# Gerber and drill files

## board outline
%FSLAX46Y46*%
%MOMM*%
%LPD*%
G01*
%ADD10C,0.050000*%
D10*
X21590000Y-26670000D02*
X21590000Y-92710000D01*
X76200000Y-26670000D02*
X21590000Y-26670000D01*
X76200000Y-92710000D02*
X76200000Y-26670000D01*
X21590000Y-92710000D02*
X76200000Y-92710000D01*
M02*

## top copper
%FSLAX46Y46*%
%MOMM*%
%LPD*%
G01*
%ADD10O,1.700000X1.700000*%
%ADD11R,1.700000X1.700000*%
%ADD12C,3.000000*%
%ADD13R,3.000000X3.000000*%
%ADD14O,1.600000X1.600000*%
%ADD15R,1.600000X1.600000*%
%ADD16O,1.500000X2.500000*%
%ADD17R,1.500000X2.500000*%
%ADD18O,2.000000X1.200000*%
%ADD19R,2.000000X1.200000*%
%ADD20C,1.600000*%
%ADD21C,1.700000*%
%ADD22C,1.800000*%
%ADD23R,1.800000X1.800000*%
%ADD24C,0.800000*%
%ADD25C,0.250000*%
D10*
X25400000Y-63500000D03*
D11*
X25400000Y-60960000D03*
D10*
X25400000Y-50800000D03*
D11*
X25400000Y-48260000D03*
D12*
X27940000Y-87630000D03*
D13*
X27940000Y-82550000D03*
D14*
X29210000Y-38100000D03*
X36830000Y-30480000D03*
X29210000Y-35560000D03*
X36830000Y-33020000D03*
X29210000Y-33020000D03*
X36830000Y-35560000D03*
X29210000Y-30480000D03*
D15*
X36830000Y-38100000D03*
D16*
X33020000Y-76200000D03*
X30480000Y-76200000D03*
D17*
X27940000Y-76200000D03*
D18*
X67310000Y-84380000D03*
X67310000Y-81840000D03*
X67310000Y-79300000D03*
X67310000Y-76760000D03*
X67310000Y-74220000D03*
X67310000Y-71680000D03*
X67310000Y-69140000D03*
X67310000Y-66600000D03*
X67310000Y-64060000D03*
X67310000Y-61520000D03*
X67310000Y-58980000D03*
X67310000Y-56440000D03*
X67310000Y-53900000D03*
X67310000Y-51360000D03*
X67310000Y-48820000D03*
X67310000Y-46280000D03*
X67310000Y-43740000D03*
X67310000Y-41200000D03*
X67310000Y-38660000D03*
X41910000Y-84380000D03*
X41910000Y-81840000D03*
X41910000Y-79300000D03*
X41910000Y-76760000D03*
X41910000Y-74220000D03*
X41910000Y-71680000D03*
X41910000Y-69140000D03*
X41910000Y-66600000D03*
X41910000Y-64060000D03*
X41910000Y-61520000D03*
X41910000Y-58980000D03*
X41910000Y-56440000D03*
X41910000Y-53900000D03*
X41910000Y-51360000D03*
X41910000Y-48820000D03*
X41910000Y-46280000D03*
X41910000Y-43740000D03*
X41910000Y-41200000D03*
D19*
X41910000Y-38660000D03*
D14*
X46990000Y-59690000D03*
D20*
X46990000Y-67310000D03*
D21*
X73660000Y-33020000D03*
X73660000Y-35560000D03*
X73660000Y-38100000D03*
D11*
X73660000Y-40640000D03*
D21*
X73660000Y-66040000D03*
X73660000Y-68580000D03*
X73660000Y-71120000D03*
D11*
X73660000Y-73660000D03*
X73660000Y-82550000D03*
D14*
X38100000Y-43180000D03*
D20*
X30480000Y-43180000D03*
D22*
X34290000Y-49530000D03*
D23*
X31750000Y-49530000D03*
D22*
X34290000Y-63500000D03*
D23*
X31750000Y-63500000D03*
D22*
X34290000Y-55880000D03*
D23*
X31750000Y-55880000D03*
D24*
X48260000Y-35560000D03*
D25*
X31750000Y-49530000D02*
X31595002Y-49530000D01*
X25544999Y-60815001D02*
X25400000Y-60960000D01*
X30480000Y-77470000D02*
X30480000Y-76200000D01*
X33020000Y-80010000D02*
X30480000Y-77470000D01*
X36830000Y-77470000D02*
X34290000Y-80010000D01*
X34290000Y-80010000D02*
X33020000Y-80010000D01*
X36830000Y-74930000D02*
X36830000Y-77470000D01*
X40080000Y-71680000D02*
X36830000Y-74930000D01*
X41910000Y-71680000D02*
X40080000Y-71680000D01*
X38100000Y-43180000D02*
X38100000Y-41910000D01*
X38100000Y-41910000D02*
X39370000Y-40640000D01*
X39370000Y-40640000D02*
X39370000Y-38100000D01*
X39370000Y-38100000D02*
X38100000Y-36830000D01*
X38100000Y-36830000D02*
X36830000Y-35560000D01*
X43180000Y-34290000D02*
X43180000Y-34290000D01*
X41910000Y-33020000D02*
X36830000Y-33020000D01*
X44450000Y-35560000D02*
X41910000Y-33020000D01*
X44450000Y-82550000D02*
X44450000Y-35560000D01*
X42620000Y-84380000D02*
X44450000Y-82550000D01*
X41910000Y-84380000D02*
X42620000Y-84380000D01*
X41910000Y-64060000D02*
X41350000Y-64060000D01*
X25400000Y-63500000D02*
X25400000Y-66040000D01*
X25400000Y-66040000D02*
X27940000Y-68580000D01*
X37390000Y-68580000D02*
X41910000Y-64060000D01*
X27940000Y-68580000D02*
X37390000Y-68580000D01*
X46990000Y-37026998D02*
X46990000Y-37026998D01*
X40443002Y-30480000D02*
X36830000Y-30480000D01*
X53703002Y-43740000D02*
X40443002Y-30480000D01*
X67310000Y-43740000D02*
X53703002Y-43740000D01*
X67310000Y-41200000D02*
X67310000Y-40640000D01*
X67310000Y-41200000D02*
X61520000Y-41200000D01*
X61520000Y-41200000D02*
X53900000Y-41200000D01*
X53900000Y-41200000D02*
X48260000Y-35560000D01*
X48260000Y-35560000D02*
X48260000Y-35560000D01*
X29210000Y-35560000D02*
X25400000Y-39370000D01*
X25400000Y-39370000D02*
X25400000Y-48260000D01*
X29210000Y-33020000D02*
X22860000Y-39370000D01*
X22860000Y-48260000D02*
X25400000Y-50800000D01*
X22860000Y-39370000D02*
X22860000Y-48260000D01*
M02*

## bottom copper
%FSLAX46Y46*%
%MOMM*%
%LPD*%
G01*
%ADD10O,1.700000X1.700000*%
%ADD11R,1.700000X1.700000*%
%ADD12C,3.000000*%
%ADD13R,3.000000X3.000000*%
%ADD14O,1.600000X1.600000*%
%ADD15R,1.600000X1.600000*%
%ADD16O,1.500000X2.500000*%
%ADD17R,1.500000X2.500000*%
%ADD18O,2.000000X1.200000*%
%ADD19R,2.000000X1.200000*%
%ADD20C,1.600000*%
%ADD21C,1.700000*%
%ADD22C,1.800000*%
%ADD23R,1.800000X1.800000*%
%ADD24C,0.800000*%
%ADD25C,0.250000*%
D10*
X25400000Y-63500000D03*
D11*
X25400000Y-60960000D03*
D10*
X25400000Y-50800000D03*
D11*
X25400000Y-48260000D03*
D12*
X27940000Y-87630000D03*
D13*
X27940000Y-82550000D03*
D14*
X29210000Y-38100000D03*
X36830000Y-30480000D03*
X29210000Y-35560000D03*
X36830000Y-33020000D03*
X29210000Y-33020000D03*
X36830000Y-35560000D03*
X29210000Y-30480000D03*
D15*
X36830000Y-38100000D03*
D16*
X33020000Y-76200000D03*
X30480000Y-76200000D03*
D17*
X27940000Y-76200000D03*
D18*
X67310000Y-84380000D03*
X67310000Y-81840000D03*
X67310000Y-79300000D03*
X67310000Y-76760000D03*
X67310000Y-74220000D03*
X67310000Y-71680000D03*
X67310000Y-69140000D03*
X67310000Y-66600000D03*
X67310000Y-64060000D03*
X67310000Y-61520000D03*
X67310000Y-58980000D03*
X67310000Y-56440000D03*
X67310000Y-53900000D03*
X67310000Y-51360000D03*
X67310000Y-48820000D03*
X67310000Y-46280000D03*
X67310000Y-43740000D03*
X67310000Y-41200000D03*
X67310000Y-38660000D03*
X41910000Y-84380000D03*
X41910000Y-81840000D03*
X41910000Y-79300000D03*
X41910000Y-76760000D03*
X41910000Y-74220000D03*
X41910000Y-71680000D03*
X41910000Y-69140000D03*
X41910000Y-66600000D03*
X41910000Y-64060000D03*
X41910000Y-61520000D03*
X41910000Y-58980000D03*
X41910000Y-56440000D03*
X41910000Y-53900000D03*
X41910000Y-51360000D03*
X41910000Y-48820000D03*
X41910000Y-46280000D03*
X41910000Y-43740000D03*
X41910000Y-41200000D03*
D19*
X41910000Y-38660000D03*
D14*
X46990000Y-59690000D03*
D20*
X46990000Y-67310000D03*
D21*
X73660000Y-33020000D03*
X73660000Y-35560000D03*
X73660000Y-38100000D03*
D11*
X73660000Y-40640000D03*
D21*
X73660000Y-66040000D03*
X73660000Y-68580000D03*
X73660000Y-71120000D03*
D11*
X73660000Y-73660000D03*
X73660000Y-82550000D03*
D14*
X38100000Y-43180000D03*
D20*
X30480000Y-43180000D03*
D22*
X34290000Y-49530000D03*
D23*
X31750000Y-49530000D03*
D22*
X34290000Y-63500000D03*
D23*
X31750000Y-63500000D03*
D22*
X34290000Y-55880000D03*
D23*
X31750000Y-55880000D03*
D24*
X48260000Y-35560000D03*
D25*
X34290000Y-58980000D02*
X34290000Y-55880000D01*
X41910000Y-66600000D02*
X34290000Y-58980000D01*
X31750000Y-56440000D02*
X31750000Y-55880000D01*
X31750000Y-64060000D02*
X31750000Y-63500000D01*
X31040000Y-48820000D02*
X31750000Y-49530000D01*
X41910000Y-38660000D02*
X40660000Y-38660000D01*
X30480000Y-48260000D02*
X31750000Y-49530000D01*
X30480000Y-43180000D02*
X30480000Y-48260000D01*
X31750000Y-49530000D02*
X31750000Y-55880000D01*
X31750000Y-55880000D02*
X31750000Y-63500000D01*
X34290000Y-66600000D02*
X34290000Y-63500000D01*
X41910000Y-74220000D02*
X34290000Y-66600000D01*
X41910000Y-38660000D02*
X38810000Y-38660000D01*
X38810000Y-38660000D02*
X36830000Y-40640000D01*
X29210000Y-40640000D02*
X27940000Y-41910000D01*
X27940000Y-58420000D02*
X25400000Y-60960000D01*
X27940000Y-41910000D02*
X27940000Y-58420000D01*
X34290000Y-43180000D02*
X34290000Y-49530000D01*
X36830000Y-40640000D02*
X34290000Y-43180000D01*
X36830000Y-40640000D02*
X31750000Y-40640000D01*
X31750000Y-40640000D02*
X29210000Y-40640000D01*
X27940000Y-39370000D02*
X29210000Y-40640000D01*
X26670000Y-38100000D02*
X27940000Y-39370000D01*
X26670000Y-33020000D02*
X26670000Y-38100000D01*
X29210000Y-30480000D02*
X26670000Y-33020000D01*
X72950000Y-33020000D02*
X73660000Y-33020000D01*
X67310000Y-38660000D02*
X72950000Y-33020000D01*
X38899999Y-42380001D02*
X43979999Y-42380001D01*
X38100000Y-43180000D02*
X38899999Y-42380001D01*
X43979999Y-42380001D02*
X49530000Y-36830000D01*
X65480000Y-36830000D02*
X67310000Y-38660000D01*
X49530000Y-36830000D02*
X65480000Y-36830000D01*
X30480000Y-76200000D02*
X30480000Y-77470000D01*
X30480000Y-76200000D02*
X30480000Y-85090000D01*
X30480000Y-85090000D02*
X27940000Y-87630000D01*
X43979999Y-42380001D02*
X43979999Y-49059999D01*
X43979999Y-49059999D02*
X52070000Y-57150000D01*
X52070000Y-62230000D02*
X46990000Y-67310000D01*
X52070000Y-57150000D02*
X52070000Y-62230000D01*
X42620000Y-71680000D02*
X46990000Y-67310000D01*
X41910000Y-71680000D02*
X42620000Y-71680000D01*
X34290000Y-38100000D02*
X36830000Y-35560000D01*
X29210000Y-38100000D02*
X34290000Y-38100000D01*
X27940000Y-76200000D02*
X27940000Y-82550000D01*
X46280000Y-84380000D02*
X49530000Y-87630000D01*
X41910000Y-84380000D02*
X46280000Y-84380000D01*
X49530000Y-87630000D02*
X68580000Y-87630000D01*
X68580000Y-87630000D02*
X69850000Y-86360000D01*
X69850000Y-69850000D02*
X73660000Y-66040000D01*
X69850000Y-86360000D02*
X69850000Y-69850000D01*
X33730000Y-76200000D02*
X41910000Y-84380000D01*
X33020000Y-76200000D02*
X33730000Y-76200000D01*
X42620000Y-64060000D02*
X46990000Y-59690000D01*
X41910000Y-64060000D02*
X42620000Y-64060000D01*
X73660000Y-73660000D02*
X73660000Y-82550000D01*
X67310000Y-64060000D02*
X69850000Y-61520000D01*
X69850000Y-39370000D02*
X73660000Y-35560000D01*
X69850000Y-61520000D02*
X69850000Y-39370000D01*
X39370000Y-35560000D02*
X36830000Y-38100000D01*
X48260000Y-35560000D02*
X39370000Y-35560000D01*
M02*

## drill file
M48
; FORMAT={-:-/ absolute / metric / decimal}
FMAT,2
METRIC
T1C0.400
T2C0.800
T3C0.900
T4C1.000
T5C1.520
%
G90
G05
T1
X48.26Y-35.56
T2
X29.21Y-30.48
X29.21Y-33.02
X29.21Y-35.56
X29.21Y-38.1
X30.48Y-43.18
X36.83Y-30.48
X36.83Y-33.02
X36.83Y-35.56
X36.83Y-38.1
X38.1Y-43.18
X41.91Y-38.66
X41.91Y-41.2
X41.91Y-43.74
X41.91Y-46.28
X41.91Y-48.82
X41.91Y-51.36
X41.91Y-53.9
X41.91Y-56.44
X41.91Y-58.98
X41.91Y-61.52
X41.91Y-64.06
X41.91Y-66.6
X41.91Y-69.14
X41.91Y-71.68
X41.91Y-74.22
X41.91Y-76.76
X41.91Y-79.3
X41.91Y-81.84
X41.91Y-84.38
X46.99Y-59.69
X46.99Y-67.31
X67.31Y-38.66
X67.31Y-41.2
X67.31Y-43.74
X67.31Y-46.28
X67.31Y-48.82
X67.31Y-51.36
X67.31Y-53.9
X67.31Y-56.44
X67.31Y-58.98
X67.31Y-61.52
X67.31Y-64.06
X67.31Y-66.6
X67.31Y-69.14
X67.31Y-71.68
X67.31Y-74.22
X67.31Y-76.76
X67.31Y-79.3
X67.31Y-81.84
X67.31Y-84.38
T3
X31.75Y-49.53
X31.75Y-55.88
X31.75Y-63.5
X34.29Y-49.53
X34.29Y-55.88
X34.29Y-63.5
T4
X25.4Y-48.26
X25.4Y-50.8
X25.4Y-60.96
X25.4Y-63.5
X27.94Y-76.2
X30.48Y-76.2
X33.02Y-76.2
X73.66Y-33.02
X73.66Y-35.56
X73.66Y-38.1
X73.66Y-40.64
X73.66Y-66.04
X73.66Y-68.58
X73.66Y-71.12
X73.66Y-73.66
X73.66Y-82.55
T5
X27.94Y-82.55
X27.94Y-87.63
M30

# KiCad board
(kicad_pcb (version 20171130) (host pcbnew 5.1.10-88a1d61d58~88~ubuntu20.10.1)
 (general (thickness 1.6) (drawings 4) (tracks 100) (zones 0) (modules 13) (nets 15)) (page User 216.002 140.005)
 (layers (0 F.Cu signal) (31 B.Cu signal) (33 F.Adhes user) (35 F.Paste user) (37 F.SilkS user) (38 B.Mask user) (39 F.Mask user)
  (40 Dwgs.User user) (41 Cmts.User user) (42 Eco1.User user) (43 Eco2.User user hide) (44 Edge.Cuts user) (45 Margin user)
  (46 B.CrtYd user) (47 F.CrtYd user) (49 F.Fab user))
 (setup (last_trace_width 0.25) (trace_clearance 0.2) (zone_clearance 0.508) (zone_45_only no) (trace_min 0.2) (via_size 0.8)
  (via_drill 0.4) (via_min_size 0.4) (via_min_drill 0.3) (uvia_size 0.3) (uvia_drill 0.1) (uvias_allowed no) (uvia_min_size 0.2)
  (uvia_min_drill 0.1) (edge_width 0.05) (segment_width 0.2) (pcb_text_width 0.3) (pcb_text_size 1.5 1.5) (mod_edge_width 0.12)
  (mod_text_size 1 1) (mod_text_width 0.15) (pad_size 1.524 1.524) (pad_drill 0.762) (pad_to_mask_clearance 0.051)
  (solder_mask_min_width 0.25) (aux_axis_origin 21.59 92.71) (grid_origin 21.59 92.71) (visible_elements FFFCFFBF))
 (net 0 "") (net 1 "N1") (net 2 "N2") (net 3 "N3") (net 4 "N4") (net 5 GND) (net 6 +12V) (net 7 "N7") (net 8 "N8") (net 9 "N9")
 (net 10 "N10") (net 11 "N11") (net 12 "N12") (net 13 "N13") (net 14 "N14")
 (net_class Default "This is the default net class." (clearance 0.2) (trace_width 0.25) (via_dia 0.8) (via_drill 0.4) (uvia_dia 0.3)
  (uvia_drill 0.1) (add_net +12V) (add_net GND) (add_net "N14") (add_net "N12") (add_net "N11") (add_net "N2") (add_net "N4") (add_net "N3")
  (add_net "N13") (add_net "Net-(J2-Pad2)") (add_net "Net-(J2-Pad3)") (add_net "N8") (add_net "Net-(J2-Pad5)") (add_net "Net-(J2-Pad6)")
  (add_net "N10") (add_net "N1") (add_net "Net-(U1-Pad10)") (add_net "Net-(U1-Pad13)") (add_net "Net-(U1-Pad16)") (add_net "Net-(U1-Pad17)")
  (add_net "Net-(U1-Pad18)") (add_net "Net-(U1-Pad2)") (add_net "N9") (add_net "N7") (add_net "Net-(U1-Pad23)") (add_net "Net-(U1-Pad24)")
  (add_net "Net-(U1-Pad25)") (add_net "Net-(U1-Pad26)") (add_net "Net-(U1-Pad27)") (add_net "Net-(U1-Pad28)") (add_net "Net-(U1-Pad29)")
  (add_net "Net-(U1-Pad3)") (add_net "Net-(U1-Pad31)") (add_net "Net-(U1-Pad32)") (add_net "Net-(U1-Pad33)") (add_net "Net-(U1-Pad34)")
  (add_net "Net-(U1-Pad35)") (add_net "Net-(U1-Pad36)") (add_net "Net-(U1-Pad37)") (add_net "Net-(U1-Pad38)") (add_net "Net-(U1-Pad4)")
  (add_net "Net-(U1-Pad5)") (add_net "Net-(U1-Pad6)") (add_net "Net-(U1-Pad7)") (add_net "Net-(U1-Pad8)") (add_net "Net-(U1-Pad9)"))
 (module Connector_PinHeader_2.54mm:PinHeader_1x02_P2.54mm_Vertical (layer F.Cu) (at 25.4 60.96)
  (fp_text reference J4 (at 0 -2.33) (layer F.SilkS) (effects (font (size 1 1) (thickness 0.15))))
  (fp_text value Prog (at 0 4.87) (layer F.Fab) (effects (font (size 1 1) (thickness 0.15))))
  (pad 2 thru_hole oval (at 0 2.54) (size 1.7 1.7) (drill 1) (layers *.Cu *.Mask) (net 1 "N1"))
  (pad 1 thru_hole rect (at 0 0) (size 1.7 1.7) (drill 1) (layers *.Cu *.Mask) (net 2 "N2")))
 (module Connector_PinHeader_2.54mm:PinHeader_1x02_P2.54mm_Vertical (layer F.Cu) (at 25.4 48.26)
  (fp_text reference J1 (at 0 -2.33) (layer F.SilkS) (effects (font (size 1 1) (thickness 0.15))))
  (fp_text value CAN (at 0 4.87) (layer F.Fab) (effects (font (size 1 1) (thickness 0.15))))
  (pad 2 thru_hole oval (at 0 2.54) (size 1.7 1.7) (drill 1) (layers *.Cu *.Mask) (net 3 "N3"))
  (pad 1 thru_hole rect (at 0 0) (size 1.7 1.7) (drill 1) (layers *.Cu *.Mask) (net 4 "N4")))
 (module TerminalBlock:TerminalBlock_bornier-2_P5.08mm (layer F.Cu) (at 27.94 82.55 270)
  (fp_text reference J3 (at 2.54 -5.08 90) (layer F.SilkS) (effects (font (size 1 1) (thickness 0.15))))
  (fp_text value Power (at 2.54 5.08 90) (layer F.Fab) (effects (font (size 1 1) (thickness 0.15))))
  (pad 2 thru_hole circle (at 5.08 0 270) (size 3 3) (drill 1.52) (layers *.Cu *.Mask) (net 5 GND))
  (pad 1 thru_hole rect (at 0 0 270) (size 3 3) (drill 1.52) (layers *.Cu *.Mask) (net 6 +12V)))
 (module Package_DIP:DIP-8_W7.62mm (layer F.Cu) (at 36.83 38.1 180)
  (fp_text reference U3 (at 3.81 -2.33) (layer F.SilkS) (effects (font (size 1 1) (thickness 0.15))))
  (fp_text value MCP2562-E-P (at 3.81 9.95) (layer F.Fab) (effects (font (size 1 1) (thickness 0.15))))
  (pad 8 thru_hole oval (at 7.62 0 180) (size 1.6 1.6) (drill 0.8) (layers *.Cu *.Mask) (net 5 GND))
  (pad 4 thru_hole oval (at 0 7.62 180) (size 1.6 1.6) (drill 0.8) (layers *.Cu *.Mask) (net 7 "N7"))
  (pad 7 thru_hole oval (at 7.62 2.54 180) (size 1.6 1.6) (drill 0.8) (layers *.Cu *.Mask) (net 4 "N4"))
  (pad 3 thru_hole oval (at 0 5.08 180) (size 1.6 1.6) (drill 0.8) (layers *.Cu *.Mask) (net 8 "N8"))
  (pad 6 thru_hole oval (at 7.62 5.08 180) (size 1.6 1.6) (drill 0.8) (layers *.Cu *.Mask) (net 3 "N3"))
  (pad 2 thru_hole oval (at 0 2.54 180) (size 1.6 1.6) (drill 0.8) (layers *.Cu *.Mask) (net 5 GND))
  (pad 5 thru_hole oval (at 7.62 7.62 180) (size 1.6 1.6) (drill 0.8) (layers *.Cu *.Mask) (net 2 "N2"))
  (pad 1 thru_hole rect (at 0 0 180) (size 1.6 1.6) (drill 0.8) (layers *.Cu *.Mask) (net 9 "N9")))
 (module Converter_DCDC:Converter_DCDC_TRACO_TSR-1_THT (layer F.Cu) (at 27.94 76.2)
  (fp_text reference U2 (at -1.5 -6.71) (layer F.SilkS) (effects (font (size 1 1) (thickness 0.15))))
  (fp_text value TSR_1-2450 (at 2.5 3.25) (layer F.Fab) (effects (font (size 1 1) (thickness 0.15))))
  (pad 3 thru_hole oval (at 5.08 0) (size 1.5 2.5) (drill 1) (layers *.Cu *.Mask) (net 8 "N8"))
  (pad 2 thru_hole oval (at 2.54 0) (size 1.5 2.5) (drill 1) (layers *.Cu *.Mask) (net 5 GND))
  (pad 1 thru_hole rect (at 0 0) (size 1.5 2.5) (drill 1) (layers *.Cu *.Mask) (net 6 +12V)))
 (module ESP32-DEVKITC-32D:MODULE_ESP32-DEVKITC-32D (layer F.Cu) (at 54.61 58.42)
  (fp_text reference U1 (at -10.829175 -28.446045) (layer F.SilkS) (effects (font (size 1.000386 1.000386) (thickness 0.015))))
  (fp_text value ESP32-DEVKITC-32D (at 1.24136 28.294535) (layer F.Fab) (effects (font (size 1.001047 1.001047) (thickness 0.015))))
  (pad 38 thru_hole oval (at 12.7 25.96) (size 2 1.2) (drill 0.8) (layers *.Cu *.Mask))
  (pad 37 thru_hole oval (at 12.7 23.42) (size 2 1.2) (drill 0.8) (layers *.Cu *.Mask))
  (pad 36 thru_hole oval (at 12.7 20.88) (size 2 1.2) (drill 0.8) (layers *.Cu *.Mask))
  (pad 35 thru_hole oval (at 12.7 18.34) (size 2 1.2) (drill 0.8) (layers *.Cu *.Mask))
  (pad 34 thru_hole oval (at 12.7 15.8) (size 2 1.2) (drill 0.8) (layers *.Cu *.Mask))
  (pad 33 thru_hole oval (at 12.7 13.26) (size 2 1.2) (drill 0.8) (layers *.Cu *.Mask))
  (pad 32 thru_hole oval (at 12.7 10.72) (size 2 1.2) (drill 0.8) (layers *.Cu *.Mask))
  (pad 31 thru_hole oval (at 12.7 8.18) (size 2 1.2) (drill 0.8) (layers *.Cu *.Mask))
  (pad 30 thru_hole oval (at 12.7 5.64) (size 2 1.2) (drill 0.8) (layers *.Cu *.Mask) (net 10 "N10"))
  (pad 29 thru_hole oval (at 12.7 3.1) (size 2 1.2) (drill 0.8) (layers *.Cu *.Mask))
  (pad 28 thru_hole oval (at 12.7 0.56) (size 2 1.2) (drill 0.8) (layers *.Cu *.Mask))
  (pad 27 thru_hole oval (at 12.7 -1.98) (size 2 1.2) (drill 0.8) (layers *.Cu *.Mask))
  (pad 26 thru_hole oval (at 12.7 -4.52) (size 2 1.2) (drill 0.8) (layers *.Cu *.Mask))
  (pad 25 thru_hole oval (at 12.7 -7.06) (size 2 1.2) (drill 0.8) (layers *.Cu *.Mask))
  (pad 24 thru_hole oval (at 12.7 -9.6) (size 2 1.2) (drill 0.8) (layers *.Cu *.Mask))
  (pad 23 thru_hole oval (at 12.7 -12.14) (size 2 1.2) (drill 0.8) (layers *.Cu *.Mask))
  (pad 22 thru_hole oval (at 12.7 -14.68) (size 2 1.2) (drill 0.8) (layers *.Cu *.Mask) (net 7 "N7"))
  (pad 21 thru_hole oval (at 12.7 -17.22) (size 2 1.2) (drill 0.8) (layers *.Cu *.Mask) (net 9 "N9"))
  (pad 20 thru_hole oval (at 12.7 -19.76) (size 2 1.2) (drill 0.8) (layers *.Cu *.Mask) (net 5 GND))
  (pad 19 thru_hole oval (at -12.7 25.96) (size 2 1.2) (drill 0.8) (layers *.Cu *.Mask) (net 8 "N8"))
  (pad 18 thru_hole oval (at -12.7 23.42) (size 2 1.2) (drill 0.8) (layers *.Cu *.Mask))
  (pad 17 thru_hole oval (at -12.7 20.88) (size 2 1.2) (drill 0.8) (layers *.Cu *.Mask))
  (pad 16 thru_hole oval (at -12.7 18.34) (size 2 1.2) (drill 0.8) (layers *.Cu *.Mask))
  (pad 15 thru_hole oval (at -12.7 15.8) (size 2 1.2) (drill 0.8) (layers *.Cu *.Mask) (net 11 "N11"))
  (pad 14 thru_hole oval (at -12.7 13.26) (size 2 1.2) (drill 0.8) (layers *.Cu *.Mask) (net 5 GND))
  (pad 13 thru_hole oval (at -12.7 10.72) (size 2 1.2) (drill 0.8) (layers *.Cu *.Mask))
  (pad 12 thru_hole oval (at -12.7 8.18) (size 2 1.2) (drill 0.8) (layers *.Cu *.Mask) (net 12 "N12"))
  (pad 11 thru_hole oval (at -12.7 5.64) (size 2 1.2) (drill 0.8) (layers *.Cu *.Mask) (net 1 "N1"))
  (pad 10 thru_hole oval (at -12.7 3.1) (size 2 1.2) (drill 0.8) (layers *.Cu *.Mask))
  (pad 9 thru_hole oval (at -12.7 0.56) (size 2 1.2) (drill 0.8) (layers *.Cu *.Mask))
  (pad 8 thru_hole oval (at -12.7 -1.98) (size 2 1.2) (drill 0.8) (layers *.Cu *.Mask))
  (pad 7 thru_hole oval (at -12.7 -4.52) (size 2 1.2) (drill 0.8) (layers *.Cu *.Mask))
  (pad 6 thru_hole oval (at -12.7 -7.06) (size 2 1.2) (drill 0.8) (layers *.Cu *.Mask))
  (pad 5 thru_hole oval (at -12.7 -9.6) (size 2 1.2) (drill 0.8) (layers *.Cu *.Mask))
  (pad 4 thru_hole oval (at -12.7 -12.14) (size 2 1.2) (drill 0.8) (layers *.Cu *.Mask))
  (pad 3 thru_hole oval (at -12.7 -14.68) (size 2 1.2) (drill 0.8) (layers *.Cu *.Mask))
  (pad 2 thru_hole oval (at -12.7 -17.22) (size 2 1.2) (drill 0.8) (layers *.Cu *.Mask))
  (pad 1 thru_hole rect (at -12.7 -19.76) (size 2 1.2) (drill 0.8) (layers *.Cu *.Mask) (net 2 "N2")))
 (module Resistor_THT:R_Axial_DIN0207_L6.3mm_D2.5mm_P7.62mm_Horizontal (layer F.Cu) (at 46.99 67.31 90)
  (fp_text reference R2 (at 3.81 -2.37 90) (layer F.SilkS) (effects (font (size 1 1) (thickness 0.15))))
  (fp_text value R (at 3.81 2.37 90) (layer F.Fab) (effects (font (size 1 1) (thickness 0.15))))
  (pad 2 thru_hole oval (at 7.62 0 90) (size 1.6 1.6) (drill 0.8) (layers *.Cu *.Mask) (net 1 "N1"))
  (pad 1 thru_hole circle (at 0 0 90) (size 1.6 1.6) (drill 0.8) (layers *.Cu *.Mask) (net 5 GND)))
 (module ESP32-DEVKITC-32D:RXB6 (layer F.Cu) (at 73.66 76.2 180)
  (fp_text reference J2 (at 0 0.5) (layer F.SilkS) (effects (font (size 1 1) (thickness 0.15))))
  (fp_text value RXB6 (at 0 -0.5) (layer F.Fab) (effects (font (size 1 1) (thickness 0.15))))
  (pad 8 thru_hole circle (at 0 43.18 180) (size 1.7 1.7) (drill 1) (layers *.Cu *.Mask) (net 5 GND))
  (pad 7 thru_hole circle (at 0 40.64 180) (size 1.7 1.7) (drill 1) (layers *.Cu *.Mask) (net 10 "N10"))
  (pad 6 thru_hole circle (at 0 38.1 180) (size 1.7 1.7) (drill 1) (layers *.Cu *.Mask))
  (pad 5 thru_hole rect (at 0 35.56 180) (size 1.7 1.7) (drill 1) (layers *.Cu *.Mask))
  (pad 4 thru_hole circle (at 0 10.16 180) (size 1.7 1.7) (drill 1) (layers *.Cu *.Mask) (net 8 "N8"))
  (pad 3 thru_hole circle (at 0 7.62 180) (size 1.7 1.7) (drill 1) (layers *.Cu *.Mask))
  (pad 2 thru_hole circle (at 0 5.08 180) (size 1.7 1.7) (drill 1) (layers *.Cu *.Mask))
  (pad 1 thru_hole rect (at 0 2.54 180) (size 1.7 1.7) (drill 1) (layers *.Cu *.Mask) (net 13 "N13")))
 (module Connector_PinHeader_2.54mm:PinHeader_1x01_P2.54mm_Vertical (layer F.Cu) (at 73.66 82.55)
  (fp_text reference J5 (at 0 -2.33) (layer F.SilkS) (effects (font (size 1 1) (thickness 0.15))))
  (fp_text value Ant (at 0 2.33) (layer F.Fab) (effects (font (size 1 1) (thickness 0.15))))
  (pad 1 thru_hole rect (at 0 0) (size 1.7 1.7) (drill 1) (layers *.Cu *.Mask) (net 13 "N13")))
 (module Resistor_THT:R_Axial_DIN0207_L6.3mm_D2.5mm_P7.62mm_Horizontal (layer F.Cu) (at 30.48 43.18)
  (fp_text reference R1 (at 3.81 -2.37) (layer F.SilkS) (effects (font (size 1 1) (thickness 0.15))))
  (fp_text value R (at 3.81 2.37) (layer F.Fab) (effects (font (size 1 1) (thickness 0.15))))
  (pad 2 thru_hole oval (at 7.62 0) (size 1.6 1.6) (drill 0.8) (layers *.Cu *.Mask) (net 5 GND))
  (pad 1 thru_hole circle (at 0 0) (size 1.6 1.6) (drill 0.8) (layers *.Cu *.Mask) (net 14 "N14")))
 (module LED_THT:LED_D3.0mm (layer F.Cu) (at 31.75 49.53)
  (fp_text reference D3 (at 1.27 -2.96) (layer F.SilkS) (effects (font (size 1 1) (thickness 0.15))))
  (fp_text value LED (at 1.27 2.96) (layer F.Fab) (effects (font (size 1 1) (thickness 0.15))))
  (pad 2 thru_hole circle (at 2.54 0) (size 1.8 1.8) (drill 0.9) (layers *.Cu *.Mask) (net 2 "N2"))
  (pad 1 thru_hole rect (at 0 0) (size 1.8 1.8) (drill 0.9) (layers *.Cu *.Mask) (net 14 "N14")))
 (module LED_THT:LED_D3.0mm (layer F.Cu) (at 31.75 63.5)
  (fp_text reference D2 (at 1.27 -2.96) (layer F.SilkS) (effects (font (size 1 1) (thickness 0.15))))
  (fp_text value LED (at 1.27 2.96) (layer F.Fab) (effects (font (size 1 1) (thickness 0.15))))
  (pad 2 thru_hole circle (at 2.54 0) (size 1.8 1.8) (drill 0.9) (layers *.Cu *.Mask) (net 11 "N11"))
  (pad 1 thru_hole rect (at 0 0) (size 1.8 1.8) (drill 0.9) (layers *.Cu *.Mask) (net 14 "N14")))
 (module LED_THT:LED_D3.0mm (layer F.Cu) (at 31.75 55.88)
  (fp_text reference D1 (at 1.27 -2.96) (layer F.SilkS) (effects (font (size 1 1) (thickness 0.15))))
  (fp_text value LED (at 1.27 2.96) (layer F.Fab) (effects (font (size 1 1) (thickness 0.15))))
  (pad 2 thru_hole circle (at 2.54 0) (size 1.8 1.8) (drill 0.9) (layers *.Cu *.Mask) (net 12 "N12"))
  (pad 1 thru_hole rect (at 0 0) (size 1.8 1.8) (drill 0.9) (layers *.Cu *.Mask) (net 14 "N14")))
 (gr_line (start 21.59 26.67) (end 21.59 92.71) (layer Edge.Cuts) (width 0.05))
 (gr_line (start 76.2 26.67) (end 21.59 26.67) (layer Edge.Cuts) (width 0.05))
 (gr_line (start 76.2 92.71) (end 76.2 26.67) (layer Edge.Cuts) (width 0.05))
 (gr_line (start 21.59 92.71) (end 76.2 92.71) (layer Edge.Cuts) (width 0.05))
 (segment (start 34.29 58.98) (end 34.29 55.88) (width 0.25) (layer B.Cu) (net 12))
 (segment (start 41.91 66.6) (end 34.29 58.98) (width 0.25) (layer B.Cu) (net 12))
 (segment (start 31.75 56.44) (end 31.75 55.88) (width 0.25) (layer B.Cu) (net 14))
 (segment (start 31.75 64.06) (end 31.75 63.5) (width 0.25) (layer B.Cu) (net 14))
 (segment (start 31.04 48.82) (end 31.75 49.53) (width 0.25) (layer B.Cu) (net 14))
 (segment (start 41.91 38.66) (end 40.66 38.66) (width 0.25) (layer B.Cu) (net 2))
 (segment (start 31.75 49.53) (end 31.595002 49.53) (width 0.25) (layer F.Cu) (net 14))
 (segment (start 30.48 48.26) (end 31.75 49.53) (width 0.25) (layer B.Cu) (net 14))
 (segment (start 30.48 43.18) (end 30.48 48.26) (width 0.25) (layer B.Cu) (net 14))
 (segment (start 31.75 49.53) (end 31.75 55.88) (width 0.25) (layer B.Cu) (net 14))
 (segment (start 31.75 55.88) (end 31.75 63.5) (width 0.25) (layer B.Cu) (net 14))
 (segment (start 34.29 66.6) (end 34.29 63.5) (width 0.25) (layer B.Cu) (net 11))
 (segment (start 41.91 74.22) (end 34.29 66.6) (width 0.25) (layer B.Cu) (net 11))
 (segment (start 25.544999 60.815001) (end 25.4 60.96) (width 0.25) (layer F.Cu) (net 2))
 (segment (start 41.91 38.66) (end 38.81 38.66) (width 0.25) (layer B.Cu) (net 2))
 (segment (start 38.81 38.66) (end 36.83 40.64) (width 0.25) (layer B.Cu) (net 2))
 (segment (start 29.21 40.64) (end 27.94 41.91) (width 0.25) (layer B.Cu) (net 2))
 (segment (start 27.94 58.42) (end 25.4 60.96) (width 0.25) (layer B.Cu) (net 2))
 (segment (start 27.94 41.91) (end 27.94 58.42) (width 0.25) (layer B.Cu) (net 2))
 (segment (start 34.29 43.18) (end 34.29 49.53) (width 0.25) (layer B.Cu) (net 2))
 (segment (start 36.83 40.64) (end 34.29 43.18) (width 0.25) (layer B.Cu) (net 2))
 (segment (start 36.83 40.64) (end 31.75 40.64) (width 0.25) (layer B.Cu) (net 2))
 (segment (start 31.75 40.64) (end 29.21 40.64) (width 0.25) (layer B.Cu) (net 2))
 (segment (start 27.94 39.37) (end 29.21 40.64) (width 0.25) (layer B.Cu) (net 2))
 (segment (start 26.67 38.1) (end 27.94 39.37) (width 0.25) (layer B.Cu) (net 2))
 (segment (start 26.67 33.02) (end 26.67 38.1) (width 0.25) (layer B.Cu) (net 2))
 (segment (start 29.21 30.48) (end 26.67 33.02) (width 0.25) (layer B.Cu) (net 2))
 (segment (start 72.95 33.02) (end 73.66 33.02) (width 0.25) (layer B.Cu) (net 5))
 (segment (start 67.31 38.66) (end 72.95 33.02) (width 0.25) (layer B.Cu) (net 5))
 (segment (start 38.899999 42.380001) (end 43.979999 42.380001) (width 0.25) (layer B.Cu) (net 5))
 (segment (start 38.1 43.18) (end 38.899999 42.380001) (width 0.25) (layer B.Cu) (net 5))
 (segment (start 43.979999 42.380001) (end 49.53 36.83) (width 0.25) (layer B.Cu) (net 5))
 (segment (start 65.48 36.83) (end 67.31 38.66) (width 0.25) (layer B.Cu) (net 5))
 (segment (start 49.53 36.83) (end 65.48 36.83) (width 0.25) (layer B.Cu) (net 5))
 (segment (start 30.48 76.2) (end 30.48 77.47) (width 0.25) (layer B.Cu) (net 5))
 (segment (start 30.48 76.2) (end 30.48 85.09) (width 0.25) (layer B.Cu) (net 5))
 (segment (start 30.48 85.09) (end 27.94 87.63) (width 0.25) (layer B.Cu) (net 5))
 (segment (start 43.979999 42.380001) (end 43.979999 49.059999) (width 0.25) (layer B.Cu) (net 5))
 (segment (start 43.979999 49.059999) (end 52.07 57.15) (width 0.25) (layer B.Cu) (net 5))
 (segment (start 52.07 62.23) (end 46.99 67.31) (width 0.25) (layer B.Cu) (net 5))
 (segment (start 52.07 57.15) (end 52.07 62.23) (width 0.25) (layer B.Cu) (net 5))
 (segment (start 42.62 71.68) (end 46.99 67.31) (width 0.25) (layer B.Cu) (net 5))
 (segment (start 41.91 71.68) (end 42.62 71.68) (width 0.25) (layer B.Cu) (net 5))
 (segment (start 30.48 77.47) (end 30.48 76.2) (width 0.25) (layer F.Cu) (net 5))
 (segment (start 33.02 80.01) (end 30.48 77.47) (width 0.25) (layer F.Cu) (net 5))
 (segment (start 36.83 77.47) (end 34.29 80.01) (width 0.25) (layer F.Cu) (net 5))
 (segment (start 34.29 80.01) (end 33.02 80.01) (width 0.25) (layer F.Cu) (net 5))
 (segment (start 36.83 74.93) (end 36.83 77.47) (width 0.25) (layer F.Cu) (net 5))
 (segment (start 40.08 71.68) (end 36.83 74.93) (width 0.25) (layer F.Cu) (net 5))
 (segment (start 41.91 71.68) (end 40.08 71.68) (width 0.25) (layer F.Cu) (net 5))
 (segment (start 34.29 38.1) (end 36.83 35.56) (width 0.25) (layer B.Cu) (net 5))
 (segment (start 29.21 38.1) (end 34.29 38.1) (width 0.25) (layer B.Cu) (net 5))
 (segment (start 38.1 43.18) (end 38.1 41.91) (width 0.25) (layer F.Cu) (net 5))
 (segment (start 38.1 41.91) (end 39.37 40.64) (width 0.25) (layer F.Cu) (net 5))
 (segment (start 39.37 40.64) (end 39.37 38.1) (width 0.25) (layer F.Cu) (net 5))
 (segment (start 39.37 38.1) (end 38.1 36.83) (width 0.25) (layer F.Cu) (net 5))
 (segment (start 38.1 36.83) (end 36.83 35.56) (width 0.25) (layer F.Cu) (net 5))
 (segment (start 27.94 76.2) (end 27.94 82.55) (width 0.25) (layer B.Cu) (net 6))
 (segment (start 46.28 84.38) (end 49.53 87.63) (width 0.25) (layer B.Cu) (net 8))
 (segment (start 41.91 84.38) (end 46.28 84.38) (width 0.25) (layer B.Cu) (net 8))
 (segment (start 49.53 87.63) (end 68.58 87.63) (width 0.25) (layer B.Cu) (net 8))
 (segment (start 68.58 87.63) (end 69.85 86.36) (width 0.25) (layer B.Cu) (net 8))
 (segment (start 69.85 69.85) (end 73.66 66.04) (width 0.25) (layer B.Cu) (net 8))
 (segment (start 69.85 86.36) (end 69.85 69.85) (width 0.25) (layer B.Cu) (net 8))
 (segment (start 43.18 34.29) (end 43.18 34.29) (width 0.25) (layer F.Cu) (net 8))
 (segment (start 33.73 76.2) (end 41.91 84.38) (width 0.25) (layer B.Cu) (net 8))
 (segment (start 33.02 76.2) (end 33.73 76.2) (width 0.25) (layer B.Cu) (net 8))
 (segment (start 41.91 33.02) (end 36.83 33.02) (width 0.25) (layer F.Cu) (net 8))
 (segment (start 44.45 35.56) (end 41.91 33.02) (width 0.25) (layer F.Cu) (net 8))
 (segment (start 44.45 82.55) (end 44.45 35.56) (width 0.25) (layer F.Cu) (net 8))
 (segment (start 42.62 84.38) (end 44.45 82.55) (width 0.25) (layer F.Cu) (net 8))
 (segment (start 41.91 84.38) (end 42.62 84.38) (width 0.25) (layer F.Cu) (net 8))
 (segment (start 42.62 64.06) (end 46.99 59.69) (width 0.25) (layer B.Cu) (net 1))
 (segment (start 41.91 64.06) (end 42.62 64.06) (width 0.25) (layer B.Cu) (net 1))
 (segment (start 41.91 64.06) (end 41.35 64.06) (width 0.25) (layer F.Cu) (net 1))
 (segment (start 25.4 63.5) (end 25.4 66.04) (width 0.25) (layer F.Cu) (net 1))
 (segment (start 25.4 66.04) (end 27.94 68.58) (width 0.25) (layer F.Cu) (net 1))
 (segment (start 37.39 68.58) (end 41.91 64.06) (width 0.25) (layer F.Cu) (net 1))
 (segment (start 27.94 68.58) (end 37.39 68.58) (width 0.25) (layer F.Cu) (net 1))
 (segment (start 73.66 73.66) (end 73.66 82.55) (width 0.25) (layer B.Cu) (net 13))
 (segment (start 67.31 64.06) (end 69.85 61.52) (width 0.25) (layer B.Cu) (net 10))
 (segment (start 69.85 39.37) (end 73.66 35.56) (width 0.25) (layer B.Cu) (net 10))
 (segment (start 69.85 61.52) (end 69.85 39.37) (width 0.25) (layer B.Cu) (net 10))
 (segment (start 46.99 37.026998) (end 46.99 37.026998) (width 0.25) (layer F.Cu) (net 7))
 (segment (start 40.443002 30.48) (end 36.83 30.48) (width 0.25) (layer F.Cu) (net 7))
 (segment (start 53.703002 43.74) (end 40.443002 30.48) (width 0.25) (layer F.Cu) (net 7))
 (segment (start 67.31 43.74) (end 53.703002 43.74) (width 0.25) (layer F.Cu) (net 7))
 (segment (start 67.31 41.2) (end 67.31 40.64) (width 0.25) (layer F.Cu) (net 9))
 (segment (start 67.31 41.2) (end 61.52 41.2) (width 0.25) (layer F.Cu) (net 9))
 (segment (start 61.52 41.2) (end 53.9 41.2) (width 0.25) (layer F.Cu) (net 9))
 (segment (start 53.9 41.2) (end 48.26 35.56) (width 0.25) (layer F.Cu) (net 9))
 (segment (start 48.26 35.56) (end 48.26 35.56) (width 0.25) (layer F.Cu) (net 9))
 (via (at 48.26 35.56) (size 0.8) (drill 0.4) (layers F.Cu B.Cu) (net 9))
 (segment (start 39.37 35.56) (end 36.83 38.1) (width 0.25) (layer B.Cu) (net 9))
 (segment (start 48.26 35.56) (end 39.37 35.56) (width 0.25) (layer B.Cu) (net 9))
 (segment (start 29.21 35.56) (end 25.4 39.37) (width 0.25) (layer F.Cu) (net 4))
 (segment (start 25.4 39.37) (end 25.4 48.26) (width 0.25) (layer F.Cu) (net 4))
 (segment (start 29.21 33.02) (end 22.86 39.37) (width 0.25) (layer F.Cu) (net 3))
 (segment (start 22.86 48.26) (end 25.4 50.8) (width 0.25) (layer F.Cu) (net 3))
 (segment (start 22.86 39.37) (end 22.86 48.26) (width 0.25) (layer F.Cu) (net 3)))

